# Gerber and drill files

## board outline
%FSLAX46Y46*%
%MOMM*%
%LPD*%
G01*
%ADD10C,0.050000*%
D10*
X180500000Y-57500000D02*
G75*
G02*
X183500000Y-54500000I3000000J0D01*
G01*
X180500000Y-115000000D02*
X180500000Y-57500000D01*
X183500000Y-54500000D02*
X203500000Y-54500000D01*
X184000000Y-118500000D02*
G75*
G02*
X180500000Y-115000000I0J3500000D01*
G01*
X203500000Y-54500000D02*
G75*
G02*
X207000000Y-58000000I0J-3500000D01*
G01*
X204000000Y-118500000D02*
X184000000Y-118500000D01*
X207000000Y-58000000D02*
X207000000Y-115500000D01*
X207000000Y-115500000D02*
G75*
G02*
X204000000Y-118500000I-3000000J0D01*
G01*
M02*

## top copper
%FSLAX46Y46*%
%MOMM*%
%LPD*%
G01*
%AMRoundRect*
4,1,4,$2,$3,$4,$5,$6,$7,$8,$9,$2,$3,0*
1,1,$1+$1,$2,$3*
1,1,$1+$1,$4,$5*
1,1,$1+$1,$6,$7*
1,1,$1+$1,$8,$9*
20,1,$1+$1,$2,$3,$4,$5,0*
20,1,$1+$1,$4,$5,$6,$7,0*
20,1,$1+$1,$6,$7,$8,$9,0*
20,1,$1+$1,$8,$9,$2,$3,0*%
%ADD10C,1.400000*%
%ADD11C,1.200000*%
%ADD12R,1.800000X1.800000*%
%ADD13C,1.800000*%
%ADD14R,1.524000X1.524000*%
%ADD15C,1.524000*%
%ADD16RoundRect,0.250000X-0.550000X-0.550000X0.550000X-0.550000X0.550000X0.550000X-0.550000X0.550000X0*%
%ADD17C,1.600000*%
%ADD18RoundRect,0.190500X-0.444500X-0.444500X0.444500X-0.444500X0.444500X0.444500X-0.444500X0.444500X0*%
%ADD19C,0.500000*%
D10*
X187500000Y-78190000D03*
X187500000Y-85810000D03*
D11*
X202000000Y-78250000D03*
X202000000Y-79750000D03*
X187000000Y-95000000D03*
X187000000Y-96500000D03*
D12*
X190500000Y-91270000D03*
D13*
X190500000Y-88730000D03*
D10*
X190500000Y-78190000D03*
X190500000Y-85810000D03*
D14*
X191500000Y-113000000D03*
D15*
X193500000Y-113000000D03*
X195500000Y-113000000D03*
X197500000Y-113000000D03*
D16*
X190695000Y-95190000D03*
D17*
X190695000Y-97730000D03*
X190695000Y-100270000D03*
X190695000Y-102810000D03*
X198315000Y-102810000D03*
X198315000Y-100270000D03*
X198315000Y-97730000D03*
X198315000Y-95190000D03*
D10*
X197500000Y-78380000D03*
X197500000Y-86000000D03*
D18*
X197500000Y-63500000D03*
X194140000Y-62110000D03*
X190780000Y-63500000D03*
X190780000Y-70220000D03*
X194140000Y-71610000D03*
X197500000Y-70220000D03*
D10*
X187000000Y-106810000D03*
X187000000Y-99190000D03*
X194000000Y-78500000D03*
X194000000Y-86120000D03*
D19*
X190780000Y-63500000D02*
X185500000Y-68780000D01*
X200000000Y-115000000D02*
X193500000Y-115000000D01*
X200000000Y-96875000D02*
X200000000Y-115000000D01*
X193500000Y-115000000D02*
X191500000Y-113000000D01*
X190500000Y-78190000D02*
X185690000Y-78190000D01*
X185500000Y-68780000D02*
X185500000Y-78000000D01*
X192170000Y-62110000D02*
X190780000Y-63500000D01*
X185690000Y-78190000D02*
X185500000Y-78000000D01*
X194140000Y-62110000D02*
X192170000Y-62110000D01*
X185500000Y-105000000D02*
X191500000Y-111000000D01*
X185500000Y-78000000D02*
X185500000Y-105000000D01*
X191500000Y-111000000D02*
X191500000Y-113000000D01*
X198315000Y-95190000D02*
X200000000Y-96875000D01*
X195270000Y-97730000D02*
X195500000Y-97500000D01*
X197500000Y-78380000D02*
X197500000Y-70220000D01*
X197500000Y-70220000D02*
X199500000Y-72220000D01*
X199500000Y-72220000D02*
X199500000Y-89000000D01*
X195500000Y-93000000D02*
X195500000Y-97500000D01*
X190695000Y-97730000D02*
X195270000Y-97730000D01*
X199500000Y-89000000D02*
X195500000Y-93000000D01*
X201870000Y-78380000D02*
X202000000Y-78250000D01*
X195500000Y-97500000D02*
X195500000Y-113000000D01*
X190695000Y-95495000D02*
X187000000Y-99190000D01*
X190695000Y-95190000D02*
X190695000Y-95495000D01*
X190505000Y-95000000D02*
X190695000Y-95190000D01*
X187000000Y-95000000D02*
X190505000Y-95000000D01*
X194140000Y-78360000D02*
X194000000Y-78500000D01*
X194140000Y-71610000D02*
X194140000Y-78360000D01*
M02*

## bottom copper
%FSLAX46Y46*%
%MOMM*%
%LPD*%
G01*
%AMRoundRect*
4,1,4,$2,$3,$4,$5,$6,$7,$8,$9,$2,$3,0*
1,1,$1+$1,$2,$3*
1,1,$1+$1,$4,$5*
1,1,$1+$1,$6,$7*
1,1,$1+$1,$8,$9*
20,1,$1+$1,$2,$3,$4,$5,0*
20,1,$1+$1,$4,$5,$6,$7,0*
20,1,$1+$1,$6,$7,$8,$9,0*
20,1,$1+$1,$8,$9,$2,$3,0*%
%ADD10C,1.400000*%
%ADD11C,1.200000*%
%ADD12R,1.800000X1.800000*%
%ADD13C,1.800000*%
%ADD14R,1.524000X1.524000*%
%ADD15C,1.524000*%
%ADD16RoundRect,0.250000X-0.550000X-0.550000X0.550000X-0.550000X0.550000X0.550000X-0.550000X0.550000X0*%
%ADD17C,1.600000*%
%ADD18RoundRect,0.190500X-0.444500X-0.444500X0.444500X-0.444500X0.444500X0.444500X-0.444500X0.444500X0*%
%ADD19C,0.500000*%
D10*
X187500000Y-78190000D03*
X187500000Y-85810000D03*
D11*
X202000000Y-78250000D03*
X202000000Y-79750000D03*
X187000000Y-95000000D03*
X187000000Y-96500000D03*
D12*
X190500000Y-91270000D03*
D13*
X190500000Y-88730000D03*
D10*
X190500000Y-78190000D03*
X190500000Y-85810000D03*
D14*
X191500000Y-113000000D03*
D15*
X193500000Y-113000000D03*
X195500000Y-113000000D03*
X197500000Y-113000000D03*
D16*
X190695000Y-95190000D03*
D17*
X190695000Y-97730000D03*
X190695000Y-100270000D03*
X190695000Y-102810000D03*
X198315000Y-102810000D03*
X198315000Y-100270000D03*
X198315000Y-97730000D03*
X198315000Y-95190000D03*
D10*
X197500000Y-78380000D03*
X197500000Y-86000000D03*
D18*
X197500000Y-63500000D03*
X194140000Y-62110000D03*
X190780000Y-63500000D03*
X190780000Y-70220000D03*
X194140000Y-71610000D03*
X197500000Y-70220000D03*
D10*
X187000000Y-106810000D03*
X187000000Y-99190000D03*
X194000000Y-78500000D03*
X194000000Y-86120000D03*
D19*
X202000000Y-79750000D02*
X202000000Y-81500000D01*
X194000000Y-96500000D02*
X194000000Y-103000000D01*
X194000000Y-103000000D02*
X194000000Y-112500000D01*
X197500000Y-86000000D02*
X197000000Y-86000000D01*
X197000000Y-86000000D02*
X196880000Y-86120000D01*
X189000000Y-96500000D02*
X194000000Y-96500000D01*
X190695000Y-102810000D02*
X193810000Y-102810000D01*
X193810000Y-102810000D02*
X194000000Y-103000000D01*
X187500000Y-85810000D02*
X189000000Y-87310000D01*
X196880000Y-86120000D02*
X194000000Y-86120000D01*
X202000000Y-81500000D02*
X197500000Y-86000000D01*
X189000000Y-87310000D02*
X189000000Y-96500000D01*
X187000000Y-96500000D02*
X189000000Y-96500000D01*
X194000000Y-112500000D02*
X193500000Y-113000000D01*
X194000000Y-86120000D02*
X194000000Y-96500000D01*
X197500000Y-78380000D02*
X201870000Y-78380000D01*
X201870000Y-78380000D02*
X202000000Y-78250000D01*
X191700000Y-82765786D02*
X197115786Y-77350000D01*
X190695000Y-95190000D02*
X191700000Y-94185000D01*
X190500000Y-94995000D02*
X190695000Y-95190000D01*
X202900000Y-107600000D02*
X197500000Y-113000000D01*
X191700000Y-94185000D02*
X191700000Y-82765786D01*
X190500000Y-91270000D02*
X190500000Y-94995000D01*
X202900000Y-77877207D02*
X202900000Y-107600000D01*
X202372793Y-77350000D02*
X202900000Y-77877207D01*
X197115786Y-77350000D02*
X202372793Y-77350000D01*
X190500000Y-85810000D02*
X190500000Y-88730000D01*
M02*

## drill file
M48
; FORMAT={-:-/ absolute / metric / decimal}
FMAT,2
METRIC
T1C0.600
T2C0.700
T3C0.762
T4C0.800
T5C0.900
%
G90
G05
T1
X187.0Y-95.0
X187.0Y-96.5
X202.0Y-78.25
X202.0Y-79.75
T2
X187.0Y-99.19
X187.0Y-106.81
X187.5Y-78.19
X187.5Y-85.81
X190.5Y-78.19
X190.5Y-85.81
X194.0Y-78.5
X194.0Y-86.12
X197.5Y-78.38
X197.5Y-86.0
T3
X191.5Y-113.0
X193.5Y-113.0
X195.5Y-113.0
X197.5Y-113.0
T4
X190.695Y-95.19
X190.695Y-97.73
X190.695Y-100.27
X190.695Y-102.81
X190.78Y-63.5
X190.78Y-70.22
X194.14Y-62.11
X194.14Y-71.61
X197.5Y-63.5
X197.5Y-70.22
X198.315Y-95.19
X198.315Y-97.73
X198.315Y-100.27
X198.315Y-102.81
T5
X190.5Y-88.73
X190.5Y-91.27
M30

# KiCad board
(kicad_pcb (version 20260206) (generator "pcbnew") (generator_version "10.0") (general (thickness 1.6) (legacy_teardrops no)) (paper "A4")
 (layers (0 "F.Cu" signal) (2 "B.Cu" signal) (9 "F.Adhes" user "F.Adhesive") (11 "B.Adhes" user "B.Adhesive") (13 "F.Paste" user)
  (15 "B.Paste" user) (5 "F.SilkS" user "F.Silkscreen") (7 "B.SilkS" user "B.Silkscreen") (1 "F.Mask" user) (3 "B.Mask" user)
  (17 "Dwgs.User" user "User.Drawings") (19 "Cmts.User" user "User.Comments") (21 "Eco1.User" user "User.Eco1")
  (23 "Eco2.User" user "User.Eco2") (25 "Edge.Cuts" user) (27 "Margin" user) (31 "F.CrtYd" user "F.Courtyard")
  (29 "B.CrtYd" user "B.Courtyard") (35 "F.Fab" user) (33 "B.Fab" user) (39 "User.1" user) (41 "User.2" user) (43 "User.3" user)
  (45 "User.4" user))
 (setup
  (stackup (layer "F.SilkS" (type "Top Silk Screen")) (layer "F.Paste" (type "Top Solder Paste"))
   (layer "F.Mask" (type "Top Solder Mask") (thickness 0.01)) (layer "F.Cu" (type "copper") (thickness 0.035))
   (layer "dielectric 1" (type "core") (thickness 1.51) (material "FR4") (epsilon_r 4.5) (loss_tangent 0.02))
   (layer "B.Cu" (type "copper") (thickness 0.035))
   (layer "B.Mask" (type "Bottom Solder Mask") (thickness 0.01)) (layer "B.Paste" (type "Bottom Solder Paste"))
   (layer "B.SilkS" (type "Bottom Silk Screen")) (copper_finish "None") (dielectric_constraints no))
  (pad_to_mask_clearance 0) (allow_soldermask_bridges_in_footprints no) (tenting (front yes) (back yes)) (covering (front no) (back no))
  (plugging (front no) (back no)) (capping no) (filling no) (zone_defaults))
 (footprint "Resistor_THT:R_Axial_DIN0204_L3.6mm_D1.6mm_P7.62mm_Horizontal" (layer "F.Cu") (at 187.5 78.19 -90)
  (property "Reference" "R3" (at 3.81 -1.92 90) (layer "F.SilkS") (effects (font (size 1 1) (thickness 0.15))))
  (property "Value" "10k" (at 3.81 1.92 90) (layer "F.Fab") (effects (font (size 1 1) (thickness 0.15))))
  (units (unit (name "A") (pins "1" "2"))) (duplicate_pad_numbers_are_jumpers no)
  (pad "1" thru_hole circle (at 0 0 270) (size 1.4 1.4) (drill 0.7) (layers "*.Cu" "*.Mask") (remove_unused_layers no) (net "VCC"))
  (pad "2" thru_hole circle (at 7.62 0 270) (size 1.4 1.4) (drill 0.7) (layers "*.Cu" "*.Mask") (remove_unused_layers no) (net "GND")))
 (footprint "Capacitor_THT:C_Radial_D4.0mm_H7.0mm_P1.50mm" (layer "F.Cu") (at 202 78.25 -90)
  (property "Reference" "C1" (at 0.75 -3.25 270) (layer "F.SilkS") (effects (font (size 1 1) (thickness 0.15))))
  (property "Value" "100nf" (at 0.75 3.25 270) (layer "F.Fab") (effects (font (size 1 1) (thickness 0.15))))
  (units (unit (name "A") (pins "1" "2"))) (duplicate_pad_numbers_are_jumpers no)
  (pad "1" thru_hole circle (at 0 0 270) (size 1.2 1.2) (drill 0.6) (layers "*.Cu" "*.Mask") (remove_unused_layers no) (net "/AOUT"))
  (pad "2" thru_hole circle (at 1.5 0 270) (size 1.2 1.2) (drill 0.6) (layers "*.Cu" "*.Mask") (remove_unused_layers no) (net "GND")))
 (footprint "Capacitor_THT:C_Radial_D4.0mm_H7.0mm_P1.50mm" (layer "F.Cu") (at 187 95 -90)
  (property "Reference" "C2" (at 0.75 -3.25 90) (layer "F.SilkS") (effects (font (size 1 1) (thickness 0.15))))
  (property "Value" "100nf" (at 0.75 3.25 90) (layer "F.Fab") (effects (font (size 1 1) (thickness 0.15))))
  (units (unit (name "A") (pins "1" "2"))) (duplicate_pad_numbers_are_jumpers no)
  (pad "1" thru_hole circle (at 0 0 270) (size 1.2 1.2) (drill 0.6) (layers "*.Cu" "*.Mask") (remove_unused_layers no) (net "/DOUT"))
  (pad "2" thru_hole circle (at 1.5 0 270) (size 1.2 1.2) (drill 0.6) (layers "*.Cu" "*.Mask") (remove_unused_layers no) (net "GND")))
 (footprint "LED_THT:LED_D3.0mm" (layer "F.Cu") (at 190.5 91.27 90)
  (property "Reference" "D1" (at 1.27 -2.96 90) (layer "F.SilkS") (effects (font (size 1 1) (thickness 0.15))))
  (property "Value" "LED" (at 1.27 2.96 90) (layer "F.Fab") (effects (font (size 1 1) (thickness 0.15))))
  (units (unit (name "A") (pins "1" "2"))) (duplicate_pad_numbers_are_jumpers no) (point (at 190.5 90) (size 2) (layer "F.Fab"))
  (pad "1" thru_hole rect (at 0 0 90) (size 1.8 1.8) (drill 0.9) (layers "*.Cu" "*.Mask") (remove_unused_layers no) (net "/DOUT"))
  (pad "2" thru_hole circle (at 2.54 0 90) (size 1.8 1.8) (drill 0.9) (layers "*.Cu" "*.Mask") (remove_unused_layers no) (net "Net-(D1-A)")))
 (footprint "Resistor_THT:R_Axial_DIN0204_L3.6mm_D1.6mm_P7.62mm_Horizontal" (layer "F.Cu") (at 190.5 78.19 -90)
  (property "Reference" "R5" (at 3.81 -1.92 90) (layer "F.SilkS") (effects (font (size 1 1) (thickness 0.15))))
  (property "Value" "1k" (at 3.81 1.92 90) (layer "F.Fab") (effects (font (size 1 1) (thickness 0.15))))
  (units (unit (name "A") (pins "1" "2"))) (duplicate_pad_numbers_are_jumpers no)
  (pad "1" thru_hole circle (at 0 0 270) (size 1.4 1.4) (drill 0.7) (layers "*.Cu" "*.Mask") (remove_unused_layers no) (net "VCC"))
  (pad "2" thru_hole circle (at 7.62 0 270) (size 1.4 1.4) (drill 0.7) (layers "*.Cu" "*.Mask") (remove_unused_layers no) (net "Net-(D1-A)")))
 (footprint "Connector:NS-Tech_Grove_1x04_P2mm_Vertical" (layer "F.Cu") (at 191.5 113 90)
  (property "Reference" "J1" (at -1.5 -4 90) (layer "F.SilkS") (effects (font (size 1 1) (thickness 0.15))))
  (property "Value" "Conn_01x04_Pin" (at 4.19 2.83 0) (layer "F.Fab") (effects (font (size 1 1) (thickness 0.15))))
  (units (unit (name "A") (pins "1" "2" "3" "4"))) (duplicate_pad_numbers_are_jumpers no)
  (pad "1" thru_hole rect (at 0 0 90) (size 1.524 1.524) (drill 0.762) (layers "*.Cu" "*.Mask") (remove_unused_layers no) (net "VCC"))
  (pad "2" thru_hole circle (at 0 2 90) (size 1.524 1.524) (drill 0.762) (layers "*.Cu" "*.Mask") (remove_unused_layers no) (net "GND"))
  (pad "3" thru_hole circle (at 0 4 90) (size 1.524 1.524) (drill 0.762) (layers "*.Cu" "*.Mask") (remove_unused_layers no) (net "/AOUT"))
  (pad "4" thru_hole circle (at 0 6 90) (size 1.524 1.524) (drill 0.762) (layers "*.Cu" "*.Mask") (remove_unused_layers no) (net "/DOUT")))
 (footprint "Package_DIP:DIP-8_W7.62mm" (layer "F.Cu") (at 190.695 95.19)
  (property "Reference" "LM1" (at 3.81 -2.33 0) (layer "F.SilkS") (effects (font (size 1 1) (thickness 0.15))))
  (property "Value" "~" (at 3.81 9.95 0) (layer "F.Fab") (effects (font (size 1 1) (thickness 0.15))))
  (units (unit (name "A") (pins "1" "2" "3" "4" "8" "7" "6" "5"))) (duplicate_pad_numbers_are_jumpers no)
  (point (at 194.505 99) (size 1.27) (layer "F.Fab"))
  (pad "1" thru_hole roundrect (at 0 0) (size 1.6 1.6) (drill 0.8) (layers "*.Cu" "*.Mask") (remove_unused_layers no)
   (roundrect_rratio 0.15625) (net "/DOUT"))
  (pad "2" thru_hole circle (at 0 2.54) (size 1.6 1.6) (drill 0.8) (layers "*.Cu" "*.Mask") (remove_unused_layers no) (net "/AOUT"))
  (pad "3" thru_hole circle (at 0 5.08) (size 1.6 1.6) (drill 0.8) (layers "*.Cu" "*.Mask") (remove_unused_layers no) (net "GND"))
  (pad "4" thru_hole circle (at 0 7.62) (size 1.6 1.6) (drill 0.8) (layers "*.Cu" "*.Mask") (remove_unused_layers no) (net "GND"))
  (pad "5" thru_hole circle (at 7.62 7.62) (size 1.6 1.6) (drill 0.8) (layers "*.Cu" "*.Mask") (remove_unused_layers no)
   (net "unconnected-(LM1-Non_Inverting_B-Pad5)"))
  (pad "6" thru_hole circle (at 7.62 5.08) (size 1.6 1.6) (drill 0.8) (layers "*.Cu" "*.Mask") (remove_unused_layers no)
   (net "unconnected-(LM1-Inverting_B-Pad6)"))
  (pad "7" thru_hole circle (at 7.62 2.54) (size 1.6 1.6) (drill 0.8) (layers "*.Cu" "*.Mask") (remove_unused_layers no)
   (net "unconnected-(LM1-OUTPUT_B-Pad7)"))
  (pad "8" thru_hole circle (at 7.62 0) (size 1.6 1.6) (drill 0.8) (layers "*.Cu" "*.Mask") (remove_unused_layers no) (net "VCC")))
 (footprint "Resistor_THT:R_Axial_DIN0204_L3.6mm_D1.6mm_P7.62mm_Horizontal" (layer "F.Cu") (at 197.5 78.38 -90)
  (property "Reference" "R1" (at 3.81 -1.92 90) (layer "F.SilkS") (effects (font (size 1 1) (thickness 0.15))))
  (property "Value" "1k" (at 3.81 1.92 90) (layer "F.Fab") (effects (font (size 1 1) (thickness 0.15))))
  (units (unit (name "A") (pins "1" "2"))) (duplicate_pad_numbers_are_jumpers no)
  (pad "1" thru_hole circle (at 0 0 270) (size 1.4 1.4) (drill 0.7) (layers "*.Cu" "*.Mask") (remove_unused_layers no) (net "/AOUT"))
  (pad "2" thru_hole circle (at 7.62 0 270) (size 1.4 1.4) (drill 0.7) (layers "*.Cu" "*.Mask") (remove_unused_layers no) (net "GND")))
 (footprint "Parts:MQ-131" (layer "F.Cu") (at 194.14 66.86)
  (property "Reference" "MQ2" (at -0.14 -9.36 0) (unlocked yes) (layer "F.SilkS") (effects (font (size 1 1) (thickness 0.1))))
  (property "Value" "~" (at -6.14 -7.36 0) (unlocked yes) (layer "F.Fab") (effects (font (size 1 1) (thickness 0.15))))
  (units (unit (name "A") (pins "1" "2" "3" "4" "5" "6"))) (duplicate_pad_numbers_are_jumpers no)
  (pad "1" thru_hole roundrect (at 3.36 -3.36) (size 1.27 1.27) (drill 0.8) (layers "*.Cu" "*.Mask") (remove_unused_layers no)
   (roundrect_rratio 0.15) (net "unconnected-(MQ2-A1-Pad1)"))
  (pad "2" thru_hole roundrect (at 0 -4.75) (size 1.27 1.27) (drill 0.8) (layers "*.Cu" "*.Mask") (remove_unused_layers no)
   (roundrect_rratio 0.15) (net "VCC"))
  (pad "3" thru_hole roundrect (at -3.36 -3.36) (size 1.27 1.27) (drill 0.8) (layers "*.Cu" "*.Mask") (remove_unused_layers no)
   (roundrect_rratio 0.15) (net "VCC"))
  (pad "4" thru_hole roundrect (at -3.36 3.36) (size 1.27 1.27) (drill 0.8) (layers "*.Cu" "*.Mask") (remove_unused_layers no)
   (roundrect_rratio 0.15) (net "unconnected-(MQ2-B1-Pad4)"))
  (pad "5" thru_hole roundrect (at 0 4.75) (size 1.27 1.27) (drill 0.8) (layers "*.Cu" "*.Mask") (remove_unused_layers no)
   (roundrect_rratio 0.15) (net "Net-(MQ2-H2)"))
  (pad "6" thru_hole roundrect (at 3.36 3.36) (size 1.27 1.27) (drill 0.8) (layers "*.Cu" "*.Mask") (remove_unused_layers no)
   (roundrect_rratio 0.15) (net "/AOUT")))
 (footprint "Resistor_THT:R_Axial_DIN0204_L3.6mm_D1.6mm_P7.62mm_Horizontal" (layer "F.Cu") (at 187 106.81 90)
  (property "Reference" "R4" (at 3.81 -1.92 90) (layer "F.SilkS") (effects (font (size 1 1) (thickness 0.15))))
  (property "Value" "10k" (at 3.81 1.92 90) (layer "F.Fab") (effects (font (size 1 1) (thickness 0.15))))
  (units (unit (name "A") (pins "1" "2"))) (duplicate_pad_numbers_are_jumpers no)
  (pad "1" thru_hole circle (at 0 0 90) (size 1.4 1.4) (drill 0.7) (layers "*.Cu" "*.Mask") (remove_unused_layers no) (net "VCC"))
  (pad "2" thru_hole circle (at 7.62 0 90) (size 1.4 1.4) (drill 0.7) (layers "*.Cu" "*.Mask") (remove_unused_layers no) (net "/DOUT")))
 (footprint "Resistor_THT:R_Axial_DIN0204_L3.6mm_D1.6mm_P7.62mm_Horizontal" (layer "F.Cu") (at 194 78.5 -90)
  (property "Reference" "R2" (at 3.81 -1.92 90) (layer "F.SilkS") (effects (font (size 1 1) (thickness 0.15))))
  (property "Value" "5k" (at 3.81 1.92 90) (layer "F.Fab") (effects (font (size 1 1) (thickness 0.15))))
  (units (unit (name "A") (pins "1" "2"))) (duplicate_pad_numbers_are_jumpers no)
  (pad "1" thru_hole circle (at 0 0 270) (size 1.4 1.4) (drill 0.7) (layers "*.Cu" "*.Mask") (remove_unused_layers no) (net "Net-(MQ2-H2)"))
  (pad "2" thru_hole circle (at 7.62 0 270) (size 1.4 1.4) (drill 0.7) (layers "*.Cu" "*.Mask") (remove_unused_layers no) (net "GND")))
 (gr_arc (start 180.5 57.5) (mid 181.37868 55.37868) (end 183.5 54.5) (stroke (width 0.05) (type default)) (layer "Edge.Cuts"))
 (gr_line (start 180.5 115) (end 180.5 57.5) (stroke (width 0.05) (type default)) (layer "Edge.Cuts"))
 (gr_line (start 183.5 54.5) (end 203.5 54.5) (stroke (width 0.05) (type default)) (layer "Edge.Cuts"))
 (gr_arc (start 184 118.5) (mid 181.525126 117.474874) (end 180.5 115) (stroke (width 0.05) (type default)) (layer "Edge.Cuts"))
 (gr_arc (start 203.5 54.5) (mid 205.974874 55.525126) (end 207 58) (stroke (width 0.05) (type default)) (layer "Edge.Cuts"))
 (gr_line (start 204 118.5) (end 184 118.5) (stroke (width 0.05) (type default)) (layer "Edge.Cuts"))
 (gr_line (start 207 58) (end 207 115.5) (stroke (width 0.05) (type default)) (layer "Edge.Cuts"))
 (gr_arc (start 207 115.5) (mid 206.12132 117.62132) (end 204 118.5) (stroke (width 0.05) (type default)) (layer "Edge.Cuts"))
 (segment (start 190.78 63.5) (end 185.5 68.78) (width 0.5) (layer "F.Cu") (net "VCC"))
 (segment (start 200 115) (end 193.5 115) (width 0.5) (layer "F.Cu") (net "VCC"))
 (segment (start 200 96.875) (end 200 115) (width 0.5) (layer "F.Cu") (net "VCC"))
 (segment (start 193.5 115) (end 191.5 113) (width 0.5) (layer "F.Cu") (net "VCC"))
 (segment (start 190.5 78.19) (end 185.69 78.19) (width 0.5) (layer "F.Cu") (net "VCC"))
 (segment (start 185.5 68.78) (end 185.5 78) (width 0.5) (layer "F.Cu") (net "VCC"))
 (segment (start 192.17 62.11) (end 190.78 63.5) (width 0.5) (layer "F.Cu") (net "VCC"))
 (segment (start 185.69 78.19) (end 185.5 78) (width 0.5) (layer "F.Cu") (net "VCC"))
 (segment (start 194.14 62.11) (end 192.17 62.11) (width 0.5) (layer "F.Cu") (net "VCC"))
 (segment (start 185.5 105) (end 191.5 111) (width 0.5) (layer "F.Cu") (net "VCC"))
 (segment (start 185.5 78) (end 185.5 105) (width 0.5) (layer "F.Cu") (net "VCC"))
 (segment (start 191.5 111) (end 191.5 113) (width 0.5) (layer "F.Cu") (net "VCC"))
 (segment (start 198.315 95.19) (end 200 96.875) (width 0.5) (layer "F.Cu") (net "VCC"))
 (segment (start 202 79.75) (end 202 81.5) (width 0.5) (layer "B.Cu") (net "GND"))
 (segment (start 194 96.5) (end 194 103) (width 0.5) (layer "B.Cu") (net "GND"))
 (segment (start 194 103) (end 194 112.5) (width 0.5) (layer "B.Cu") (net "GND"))
 (segment (start 197.5 86) (end 197 86) (width 0.5) (layer "B.Cu") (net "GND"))
 (segment (start 197 86) (end 196.88 86.12) (width 0.5) (layer "B.Cu") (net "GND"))
 (segment (start 189 96.5) (end 194 96.5) (width 0.5) (layer "B.Cu") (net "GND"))
 (segment (start 190.695 102.81) (end 193.81 102.81) (width 0.5) (layer "B.Cu") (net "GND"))
 (segment (start 193.81 102.81) (end 194 103) (width 0.5) (layer "B.Cu") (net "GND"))
 (segment (start 187.5 85.81) (end 189 87.31) (width 0.5) (layer "B.Cu") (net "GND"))
 (segment (start 196.88 86.12) (end 194 86.12) (width 0.5) (layer "B.Cu") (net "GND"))
 (segment (start 202 81.5) (end 197.5 86) (width 0.5) (layer "B.Cu") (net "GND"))
 (segment (start 189 87.31) (end 189 96.5) (width 0.5) (layer "B.Cu") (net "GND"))
 (segment (start 187 96.5) (end 189 96.5) (width 0.5) (layer "B.Cu") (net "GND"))
 (segment (start 194 112.5) (end 193.5 113) (width 0.5) (layer "B.Cu") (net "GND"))
 (segment (start 194 86.12) (end 194 96.5) (width 0.5) (layer "B.Cu") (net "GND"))
 (segment (start 195.27 97.73) (end 195.5 97.5) (width 0.5) (layer "F.Cu") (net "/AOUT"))
 (segment (start 197.5 78.38) (end 197.5 70.22) (width 0.5) (layer "F.Cu") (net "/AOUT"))
 (segment (start 197.5 70.22) (end 199.5 72.22) (width 0.5) (layer "F.Cu") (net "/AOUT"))
 (segment (start 199.5 72.22) (end 199.5 89) (width 0.5) (layer "F.Cu") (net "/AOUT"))
 (segment (start 195.5 93) (end 195.5 97.5) (width 0.5) (layer "F.Cu") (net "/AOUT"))
 (segment (start 190.695 97.73) (end 195.27 97.73) (width 0.5) (layer "F.Cu") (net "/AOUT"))
 (segment (start 199.5 89) (end 195.5 93) (width 0.5) (layer "F.Cu") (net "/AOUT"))
 (segment (start 201.87 78.38) (end 202 78.25) (width 0.5) (layer "F.Cu") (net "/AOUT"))
 (segment (start 195.5 97.5) (end 195.5 113) (width 0.5) (layer "F.Cu") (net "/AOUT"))
 (segment (start 197.5 78.38) (end 201.87 78.38) (width 0.5) (layer "B.Cu") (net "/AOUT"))
 (segment (start 201.87 78.38) (end 202 78.25) (width 0.5) (layer "B.Cu") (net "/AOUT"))
 (segment (start 190.695 95.495) (end 187 99.19) (width 0.5) (layer "F.Cu") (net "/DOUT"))
 (segment (start 190.695 95.19) (end 190.695 95.495) (width 0.5) (layer "F.Cu") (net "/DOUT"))
 (segment (start 190.505 95) (end 190.695 95.19) (width 0.5) (layer "F.Cu") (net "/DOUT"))
 (segment (start 187 95) (end 190.505 95) (width 0.5) (layer "F.Cu") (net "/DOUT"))
 (segment (start 191.7 82.765786) (end 197.115786 77.35) (width 0.5) (layer "B.Cu") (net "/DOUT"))
 (segment (start 190.695 95.19) (end 191.7 94.185) (width 0.5) (layer "B.Cu") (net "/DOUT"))
 (segment (start 190.5 94.995) (end 190.695 95.19) (width 0.5) (layer "B.Cu") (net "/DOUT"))
 (segment (start 202.9 107.6) (end 197.5 113) (width 0.5) (layer "B.Cu") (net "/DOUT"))
 (segment (start 191.7 94.185) (end 191.7 82.765786) (width 0.5) (layer "B.Cu") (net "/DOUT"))
 (segment (start 190.5 91.27) (end 190.5 94.995) (width 0.5) (layer "B.Cu") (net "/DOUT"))
 (segment (start 202.9 77.877207) (end 202.9 107.6) (width 0.5) (layer "B.Cu") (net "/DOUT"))
 (segment (start 202.372793 77.35) (end 202.9 77.877207) (width 0.5) (layer "B.Cu") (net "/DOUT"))
 (segment (start 197.115786 77.35) (end 202.372793 77.35) (width 0.5) (layer "B.Cu") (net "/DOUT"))
 (segment (start 190.5 85.81) (end 190.5 88.73) (width 0.5) (layer "B.Cu") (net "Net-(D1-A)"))
 (segment (start 194.14 78.36) (end 194 78.5) (width 0.5) (layer "F.Cu") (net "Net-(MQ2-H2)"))
 (segment (start 194.14 71.61) (end 194.14 78.36) (width 0.5) (layer "F.Cu") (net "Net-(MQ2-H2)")))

